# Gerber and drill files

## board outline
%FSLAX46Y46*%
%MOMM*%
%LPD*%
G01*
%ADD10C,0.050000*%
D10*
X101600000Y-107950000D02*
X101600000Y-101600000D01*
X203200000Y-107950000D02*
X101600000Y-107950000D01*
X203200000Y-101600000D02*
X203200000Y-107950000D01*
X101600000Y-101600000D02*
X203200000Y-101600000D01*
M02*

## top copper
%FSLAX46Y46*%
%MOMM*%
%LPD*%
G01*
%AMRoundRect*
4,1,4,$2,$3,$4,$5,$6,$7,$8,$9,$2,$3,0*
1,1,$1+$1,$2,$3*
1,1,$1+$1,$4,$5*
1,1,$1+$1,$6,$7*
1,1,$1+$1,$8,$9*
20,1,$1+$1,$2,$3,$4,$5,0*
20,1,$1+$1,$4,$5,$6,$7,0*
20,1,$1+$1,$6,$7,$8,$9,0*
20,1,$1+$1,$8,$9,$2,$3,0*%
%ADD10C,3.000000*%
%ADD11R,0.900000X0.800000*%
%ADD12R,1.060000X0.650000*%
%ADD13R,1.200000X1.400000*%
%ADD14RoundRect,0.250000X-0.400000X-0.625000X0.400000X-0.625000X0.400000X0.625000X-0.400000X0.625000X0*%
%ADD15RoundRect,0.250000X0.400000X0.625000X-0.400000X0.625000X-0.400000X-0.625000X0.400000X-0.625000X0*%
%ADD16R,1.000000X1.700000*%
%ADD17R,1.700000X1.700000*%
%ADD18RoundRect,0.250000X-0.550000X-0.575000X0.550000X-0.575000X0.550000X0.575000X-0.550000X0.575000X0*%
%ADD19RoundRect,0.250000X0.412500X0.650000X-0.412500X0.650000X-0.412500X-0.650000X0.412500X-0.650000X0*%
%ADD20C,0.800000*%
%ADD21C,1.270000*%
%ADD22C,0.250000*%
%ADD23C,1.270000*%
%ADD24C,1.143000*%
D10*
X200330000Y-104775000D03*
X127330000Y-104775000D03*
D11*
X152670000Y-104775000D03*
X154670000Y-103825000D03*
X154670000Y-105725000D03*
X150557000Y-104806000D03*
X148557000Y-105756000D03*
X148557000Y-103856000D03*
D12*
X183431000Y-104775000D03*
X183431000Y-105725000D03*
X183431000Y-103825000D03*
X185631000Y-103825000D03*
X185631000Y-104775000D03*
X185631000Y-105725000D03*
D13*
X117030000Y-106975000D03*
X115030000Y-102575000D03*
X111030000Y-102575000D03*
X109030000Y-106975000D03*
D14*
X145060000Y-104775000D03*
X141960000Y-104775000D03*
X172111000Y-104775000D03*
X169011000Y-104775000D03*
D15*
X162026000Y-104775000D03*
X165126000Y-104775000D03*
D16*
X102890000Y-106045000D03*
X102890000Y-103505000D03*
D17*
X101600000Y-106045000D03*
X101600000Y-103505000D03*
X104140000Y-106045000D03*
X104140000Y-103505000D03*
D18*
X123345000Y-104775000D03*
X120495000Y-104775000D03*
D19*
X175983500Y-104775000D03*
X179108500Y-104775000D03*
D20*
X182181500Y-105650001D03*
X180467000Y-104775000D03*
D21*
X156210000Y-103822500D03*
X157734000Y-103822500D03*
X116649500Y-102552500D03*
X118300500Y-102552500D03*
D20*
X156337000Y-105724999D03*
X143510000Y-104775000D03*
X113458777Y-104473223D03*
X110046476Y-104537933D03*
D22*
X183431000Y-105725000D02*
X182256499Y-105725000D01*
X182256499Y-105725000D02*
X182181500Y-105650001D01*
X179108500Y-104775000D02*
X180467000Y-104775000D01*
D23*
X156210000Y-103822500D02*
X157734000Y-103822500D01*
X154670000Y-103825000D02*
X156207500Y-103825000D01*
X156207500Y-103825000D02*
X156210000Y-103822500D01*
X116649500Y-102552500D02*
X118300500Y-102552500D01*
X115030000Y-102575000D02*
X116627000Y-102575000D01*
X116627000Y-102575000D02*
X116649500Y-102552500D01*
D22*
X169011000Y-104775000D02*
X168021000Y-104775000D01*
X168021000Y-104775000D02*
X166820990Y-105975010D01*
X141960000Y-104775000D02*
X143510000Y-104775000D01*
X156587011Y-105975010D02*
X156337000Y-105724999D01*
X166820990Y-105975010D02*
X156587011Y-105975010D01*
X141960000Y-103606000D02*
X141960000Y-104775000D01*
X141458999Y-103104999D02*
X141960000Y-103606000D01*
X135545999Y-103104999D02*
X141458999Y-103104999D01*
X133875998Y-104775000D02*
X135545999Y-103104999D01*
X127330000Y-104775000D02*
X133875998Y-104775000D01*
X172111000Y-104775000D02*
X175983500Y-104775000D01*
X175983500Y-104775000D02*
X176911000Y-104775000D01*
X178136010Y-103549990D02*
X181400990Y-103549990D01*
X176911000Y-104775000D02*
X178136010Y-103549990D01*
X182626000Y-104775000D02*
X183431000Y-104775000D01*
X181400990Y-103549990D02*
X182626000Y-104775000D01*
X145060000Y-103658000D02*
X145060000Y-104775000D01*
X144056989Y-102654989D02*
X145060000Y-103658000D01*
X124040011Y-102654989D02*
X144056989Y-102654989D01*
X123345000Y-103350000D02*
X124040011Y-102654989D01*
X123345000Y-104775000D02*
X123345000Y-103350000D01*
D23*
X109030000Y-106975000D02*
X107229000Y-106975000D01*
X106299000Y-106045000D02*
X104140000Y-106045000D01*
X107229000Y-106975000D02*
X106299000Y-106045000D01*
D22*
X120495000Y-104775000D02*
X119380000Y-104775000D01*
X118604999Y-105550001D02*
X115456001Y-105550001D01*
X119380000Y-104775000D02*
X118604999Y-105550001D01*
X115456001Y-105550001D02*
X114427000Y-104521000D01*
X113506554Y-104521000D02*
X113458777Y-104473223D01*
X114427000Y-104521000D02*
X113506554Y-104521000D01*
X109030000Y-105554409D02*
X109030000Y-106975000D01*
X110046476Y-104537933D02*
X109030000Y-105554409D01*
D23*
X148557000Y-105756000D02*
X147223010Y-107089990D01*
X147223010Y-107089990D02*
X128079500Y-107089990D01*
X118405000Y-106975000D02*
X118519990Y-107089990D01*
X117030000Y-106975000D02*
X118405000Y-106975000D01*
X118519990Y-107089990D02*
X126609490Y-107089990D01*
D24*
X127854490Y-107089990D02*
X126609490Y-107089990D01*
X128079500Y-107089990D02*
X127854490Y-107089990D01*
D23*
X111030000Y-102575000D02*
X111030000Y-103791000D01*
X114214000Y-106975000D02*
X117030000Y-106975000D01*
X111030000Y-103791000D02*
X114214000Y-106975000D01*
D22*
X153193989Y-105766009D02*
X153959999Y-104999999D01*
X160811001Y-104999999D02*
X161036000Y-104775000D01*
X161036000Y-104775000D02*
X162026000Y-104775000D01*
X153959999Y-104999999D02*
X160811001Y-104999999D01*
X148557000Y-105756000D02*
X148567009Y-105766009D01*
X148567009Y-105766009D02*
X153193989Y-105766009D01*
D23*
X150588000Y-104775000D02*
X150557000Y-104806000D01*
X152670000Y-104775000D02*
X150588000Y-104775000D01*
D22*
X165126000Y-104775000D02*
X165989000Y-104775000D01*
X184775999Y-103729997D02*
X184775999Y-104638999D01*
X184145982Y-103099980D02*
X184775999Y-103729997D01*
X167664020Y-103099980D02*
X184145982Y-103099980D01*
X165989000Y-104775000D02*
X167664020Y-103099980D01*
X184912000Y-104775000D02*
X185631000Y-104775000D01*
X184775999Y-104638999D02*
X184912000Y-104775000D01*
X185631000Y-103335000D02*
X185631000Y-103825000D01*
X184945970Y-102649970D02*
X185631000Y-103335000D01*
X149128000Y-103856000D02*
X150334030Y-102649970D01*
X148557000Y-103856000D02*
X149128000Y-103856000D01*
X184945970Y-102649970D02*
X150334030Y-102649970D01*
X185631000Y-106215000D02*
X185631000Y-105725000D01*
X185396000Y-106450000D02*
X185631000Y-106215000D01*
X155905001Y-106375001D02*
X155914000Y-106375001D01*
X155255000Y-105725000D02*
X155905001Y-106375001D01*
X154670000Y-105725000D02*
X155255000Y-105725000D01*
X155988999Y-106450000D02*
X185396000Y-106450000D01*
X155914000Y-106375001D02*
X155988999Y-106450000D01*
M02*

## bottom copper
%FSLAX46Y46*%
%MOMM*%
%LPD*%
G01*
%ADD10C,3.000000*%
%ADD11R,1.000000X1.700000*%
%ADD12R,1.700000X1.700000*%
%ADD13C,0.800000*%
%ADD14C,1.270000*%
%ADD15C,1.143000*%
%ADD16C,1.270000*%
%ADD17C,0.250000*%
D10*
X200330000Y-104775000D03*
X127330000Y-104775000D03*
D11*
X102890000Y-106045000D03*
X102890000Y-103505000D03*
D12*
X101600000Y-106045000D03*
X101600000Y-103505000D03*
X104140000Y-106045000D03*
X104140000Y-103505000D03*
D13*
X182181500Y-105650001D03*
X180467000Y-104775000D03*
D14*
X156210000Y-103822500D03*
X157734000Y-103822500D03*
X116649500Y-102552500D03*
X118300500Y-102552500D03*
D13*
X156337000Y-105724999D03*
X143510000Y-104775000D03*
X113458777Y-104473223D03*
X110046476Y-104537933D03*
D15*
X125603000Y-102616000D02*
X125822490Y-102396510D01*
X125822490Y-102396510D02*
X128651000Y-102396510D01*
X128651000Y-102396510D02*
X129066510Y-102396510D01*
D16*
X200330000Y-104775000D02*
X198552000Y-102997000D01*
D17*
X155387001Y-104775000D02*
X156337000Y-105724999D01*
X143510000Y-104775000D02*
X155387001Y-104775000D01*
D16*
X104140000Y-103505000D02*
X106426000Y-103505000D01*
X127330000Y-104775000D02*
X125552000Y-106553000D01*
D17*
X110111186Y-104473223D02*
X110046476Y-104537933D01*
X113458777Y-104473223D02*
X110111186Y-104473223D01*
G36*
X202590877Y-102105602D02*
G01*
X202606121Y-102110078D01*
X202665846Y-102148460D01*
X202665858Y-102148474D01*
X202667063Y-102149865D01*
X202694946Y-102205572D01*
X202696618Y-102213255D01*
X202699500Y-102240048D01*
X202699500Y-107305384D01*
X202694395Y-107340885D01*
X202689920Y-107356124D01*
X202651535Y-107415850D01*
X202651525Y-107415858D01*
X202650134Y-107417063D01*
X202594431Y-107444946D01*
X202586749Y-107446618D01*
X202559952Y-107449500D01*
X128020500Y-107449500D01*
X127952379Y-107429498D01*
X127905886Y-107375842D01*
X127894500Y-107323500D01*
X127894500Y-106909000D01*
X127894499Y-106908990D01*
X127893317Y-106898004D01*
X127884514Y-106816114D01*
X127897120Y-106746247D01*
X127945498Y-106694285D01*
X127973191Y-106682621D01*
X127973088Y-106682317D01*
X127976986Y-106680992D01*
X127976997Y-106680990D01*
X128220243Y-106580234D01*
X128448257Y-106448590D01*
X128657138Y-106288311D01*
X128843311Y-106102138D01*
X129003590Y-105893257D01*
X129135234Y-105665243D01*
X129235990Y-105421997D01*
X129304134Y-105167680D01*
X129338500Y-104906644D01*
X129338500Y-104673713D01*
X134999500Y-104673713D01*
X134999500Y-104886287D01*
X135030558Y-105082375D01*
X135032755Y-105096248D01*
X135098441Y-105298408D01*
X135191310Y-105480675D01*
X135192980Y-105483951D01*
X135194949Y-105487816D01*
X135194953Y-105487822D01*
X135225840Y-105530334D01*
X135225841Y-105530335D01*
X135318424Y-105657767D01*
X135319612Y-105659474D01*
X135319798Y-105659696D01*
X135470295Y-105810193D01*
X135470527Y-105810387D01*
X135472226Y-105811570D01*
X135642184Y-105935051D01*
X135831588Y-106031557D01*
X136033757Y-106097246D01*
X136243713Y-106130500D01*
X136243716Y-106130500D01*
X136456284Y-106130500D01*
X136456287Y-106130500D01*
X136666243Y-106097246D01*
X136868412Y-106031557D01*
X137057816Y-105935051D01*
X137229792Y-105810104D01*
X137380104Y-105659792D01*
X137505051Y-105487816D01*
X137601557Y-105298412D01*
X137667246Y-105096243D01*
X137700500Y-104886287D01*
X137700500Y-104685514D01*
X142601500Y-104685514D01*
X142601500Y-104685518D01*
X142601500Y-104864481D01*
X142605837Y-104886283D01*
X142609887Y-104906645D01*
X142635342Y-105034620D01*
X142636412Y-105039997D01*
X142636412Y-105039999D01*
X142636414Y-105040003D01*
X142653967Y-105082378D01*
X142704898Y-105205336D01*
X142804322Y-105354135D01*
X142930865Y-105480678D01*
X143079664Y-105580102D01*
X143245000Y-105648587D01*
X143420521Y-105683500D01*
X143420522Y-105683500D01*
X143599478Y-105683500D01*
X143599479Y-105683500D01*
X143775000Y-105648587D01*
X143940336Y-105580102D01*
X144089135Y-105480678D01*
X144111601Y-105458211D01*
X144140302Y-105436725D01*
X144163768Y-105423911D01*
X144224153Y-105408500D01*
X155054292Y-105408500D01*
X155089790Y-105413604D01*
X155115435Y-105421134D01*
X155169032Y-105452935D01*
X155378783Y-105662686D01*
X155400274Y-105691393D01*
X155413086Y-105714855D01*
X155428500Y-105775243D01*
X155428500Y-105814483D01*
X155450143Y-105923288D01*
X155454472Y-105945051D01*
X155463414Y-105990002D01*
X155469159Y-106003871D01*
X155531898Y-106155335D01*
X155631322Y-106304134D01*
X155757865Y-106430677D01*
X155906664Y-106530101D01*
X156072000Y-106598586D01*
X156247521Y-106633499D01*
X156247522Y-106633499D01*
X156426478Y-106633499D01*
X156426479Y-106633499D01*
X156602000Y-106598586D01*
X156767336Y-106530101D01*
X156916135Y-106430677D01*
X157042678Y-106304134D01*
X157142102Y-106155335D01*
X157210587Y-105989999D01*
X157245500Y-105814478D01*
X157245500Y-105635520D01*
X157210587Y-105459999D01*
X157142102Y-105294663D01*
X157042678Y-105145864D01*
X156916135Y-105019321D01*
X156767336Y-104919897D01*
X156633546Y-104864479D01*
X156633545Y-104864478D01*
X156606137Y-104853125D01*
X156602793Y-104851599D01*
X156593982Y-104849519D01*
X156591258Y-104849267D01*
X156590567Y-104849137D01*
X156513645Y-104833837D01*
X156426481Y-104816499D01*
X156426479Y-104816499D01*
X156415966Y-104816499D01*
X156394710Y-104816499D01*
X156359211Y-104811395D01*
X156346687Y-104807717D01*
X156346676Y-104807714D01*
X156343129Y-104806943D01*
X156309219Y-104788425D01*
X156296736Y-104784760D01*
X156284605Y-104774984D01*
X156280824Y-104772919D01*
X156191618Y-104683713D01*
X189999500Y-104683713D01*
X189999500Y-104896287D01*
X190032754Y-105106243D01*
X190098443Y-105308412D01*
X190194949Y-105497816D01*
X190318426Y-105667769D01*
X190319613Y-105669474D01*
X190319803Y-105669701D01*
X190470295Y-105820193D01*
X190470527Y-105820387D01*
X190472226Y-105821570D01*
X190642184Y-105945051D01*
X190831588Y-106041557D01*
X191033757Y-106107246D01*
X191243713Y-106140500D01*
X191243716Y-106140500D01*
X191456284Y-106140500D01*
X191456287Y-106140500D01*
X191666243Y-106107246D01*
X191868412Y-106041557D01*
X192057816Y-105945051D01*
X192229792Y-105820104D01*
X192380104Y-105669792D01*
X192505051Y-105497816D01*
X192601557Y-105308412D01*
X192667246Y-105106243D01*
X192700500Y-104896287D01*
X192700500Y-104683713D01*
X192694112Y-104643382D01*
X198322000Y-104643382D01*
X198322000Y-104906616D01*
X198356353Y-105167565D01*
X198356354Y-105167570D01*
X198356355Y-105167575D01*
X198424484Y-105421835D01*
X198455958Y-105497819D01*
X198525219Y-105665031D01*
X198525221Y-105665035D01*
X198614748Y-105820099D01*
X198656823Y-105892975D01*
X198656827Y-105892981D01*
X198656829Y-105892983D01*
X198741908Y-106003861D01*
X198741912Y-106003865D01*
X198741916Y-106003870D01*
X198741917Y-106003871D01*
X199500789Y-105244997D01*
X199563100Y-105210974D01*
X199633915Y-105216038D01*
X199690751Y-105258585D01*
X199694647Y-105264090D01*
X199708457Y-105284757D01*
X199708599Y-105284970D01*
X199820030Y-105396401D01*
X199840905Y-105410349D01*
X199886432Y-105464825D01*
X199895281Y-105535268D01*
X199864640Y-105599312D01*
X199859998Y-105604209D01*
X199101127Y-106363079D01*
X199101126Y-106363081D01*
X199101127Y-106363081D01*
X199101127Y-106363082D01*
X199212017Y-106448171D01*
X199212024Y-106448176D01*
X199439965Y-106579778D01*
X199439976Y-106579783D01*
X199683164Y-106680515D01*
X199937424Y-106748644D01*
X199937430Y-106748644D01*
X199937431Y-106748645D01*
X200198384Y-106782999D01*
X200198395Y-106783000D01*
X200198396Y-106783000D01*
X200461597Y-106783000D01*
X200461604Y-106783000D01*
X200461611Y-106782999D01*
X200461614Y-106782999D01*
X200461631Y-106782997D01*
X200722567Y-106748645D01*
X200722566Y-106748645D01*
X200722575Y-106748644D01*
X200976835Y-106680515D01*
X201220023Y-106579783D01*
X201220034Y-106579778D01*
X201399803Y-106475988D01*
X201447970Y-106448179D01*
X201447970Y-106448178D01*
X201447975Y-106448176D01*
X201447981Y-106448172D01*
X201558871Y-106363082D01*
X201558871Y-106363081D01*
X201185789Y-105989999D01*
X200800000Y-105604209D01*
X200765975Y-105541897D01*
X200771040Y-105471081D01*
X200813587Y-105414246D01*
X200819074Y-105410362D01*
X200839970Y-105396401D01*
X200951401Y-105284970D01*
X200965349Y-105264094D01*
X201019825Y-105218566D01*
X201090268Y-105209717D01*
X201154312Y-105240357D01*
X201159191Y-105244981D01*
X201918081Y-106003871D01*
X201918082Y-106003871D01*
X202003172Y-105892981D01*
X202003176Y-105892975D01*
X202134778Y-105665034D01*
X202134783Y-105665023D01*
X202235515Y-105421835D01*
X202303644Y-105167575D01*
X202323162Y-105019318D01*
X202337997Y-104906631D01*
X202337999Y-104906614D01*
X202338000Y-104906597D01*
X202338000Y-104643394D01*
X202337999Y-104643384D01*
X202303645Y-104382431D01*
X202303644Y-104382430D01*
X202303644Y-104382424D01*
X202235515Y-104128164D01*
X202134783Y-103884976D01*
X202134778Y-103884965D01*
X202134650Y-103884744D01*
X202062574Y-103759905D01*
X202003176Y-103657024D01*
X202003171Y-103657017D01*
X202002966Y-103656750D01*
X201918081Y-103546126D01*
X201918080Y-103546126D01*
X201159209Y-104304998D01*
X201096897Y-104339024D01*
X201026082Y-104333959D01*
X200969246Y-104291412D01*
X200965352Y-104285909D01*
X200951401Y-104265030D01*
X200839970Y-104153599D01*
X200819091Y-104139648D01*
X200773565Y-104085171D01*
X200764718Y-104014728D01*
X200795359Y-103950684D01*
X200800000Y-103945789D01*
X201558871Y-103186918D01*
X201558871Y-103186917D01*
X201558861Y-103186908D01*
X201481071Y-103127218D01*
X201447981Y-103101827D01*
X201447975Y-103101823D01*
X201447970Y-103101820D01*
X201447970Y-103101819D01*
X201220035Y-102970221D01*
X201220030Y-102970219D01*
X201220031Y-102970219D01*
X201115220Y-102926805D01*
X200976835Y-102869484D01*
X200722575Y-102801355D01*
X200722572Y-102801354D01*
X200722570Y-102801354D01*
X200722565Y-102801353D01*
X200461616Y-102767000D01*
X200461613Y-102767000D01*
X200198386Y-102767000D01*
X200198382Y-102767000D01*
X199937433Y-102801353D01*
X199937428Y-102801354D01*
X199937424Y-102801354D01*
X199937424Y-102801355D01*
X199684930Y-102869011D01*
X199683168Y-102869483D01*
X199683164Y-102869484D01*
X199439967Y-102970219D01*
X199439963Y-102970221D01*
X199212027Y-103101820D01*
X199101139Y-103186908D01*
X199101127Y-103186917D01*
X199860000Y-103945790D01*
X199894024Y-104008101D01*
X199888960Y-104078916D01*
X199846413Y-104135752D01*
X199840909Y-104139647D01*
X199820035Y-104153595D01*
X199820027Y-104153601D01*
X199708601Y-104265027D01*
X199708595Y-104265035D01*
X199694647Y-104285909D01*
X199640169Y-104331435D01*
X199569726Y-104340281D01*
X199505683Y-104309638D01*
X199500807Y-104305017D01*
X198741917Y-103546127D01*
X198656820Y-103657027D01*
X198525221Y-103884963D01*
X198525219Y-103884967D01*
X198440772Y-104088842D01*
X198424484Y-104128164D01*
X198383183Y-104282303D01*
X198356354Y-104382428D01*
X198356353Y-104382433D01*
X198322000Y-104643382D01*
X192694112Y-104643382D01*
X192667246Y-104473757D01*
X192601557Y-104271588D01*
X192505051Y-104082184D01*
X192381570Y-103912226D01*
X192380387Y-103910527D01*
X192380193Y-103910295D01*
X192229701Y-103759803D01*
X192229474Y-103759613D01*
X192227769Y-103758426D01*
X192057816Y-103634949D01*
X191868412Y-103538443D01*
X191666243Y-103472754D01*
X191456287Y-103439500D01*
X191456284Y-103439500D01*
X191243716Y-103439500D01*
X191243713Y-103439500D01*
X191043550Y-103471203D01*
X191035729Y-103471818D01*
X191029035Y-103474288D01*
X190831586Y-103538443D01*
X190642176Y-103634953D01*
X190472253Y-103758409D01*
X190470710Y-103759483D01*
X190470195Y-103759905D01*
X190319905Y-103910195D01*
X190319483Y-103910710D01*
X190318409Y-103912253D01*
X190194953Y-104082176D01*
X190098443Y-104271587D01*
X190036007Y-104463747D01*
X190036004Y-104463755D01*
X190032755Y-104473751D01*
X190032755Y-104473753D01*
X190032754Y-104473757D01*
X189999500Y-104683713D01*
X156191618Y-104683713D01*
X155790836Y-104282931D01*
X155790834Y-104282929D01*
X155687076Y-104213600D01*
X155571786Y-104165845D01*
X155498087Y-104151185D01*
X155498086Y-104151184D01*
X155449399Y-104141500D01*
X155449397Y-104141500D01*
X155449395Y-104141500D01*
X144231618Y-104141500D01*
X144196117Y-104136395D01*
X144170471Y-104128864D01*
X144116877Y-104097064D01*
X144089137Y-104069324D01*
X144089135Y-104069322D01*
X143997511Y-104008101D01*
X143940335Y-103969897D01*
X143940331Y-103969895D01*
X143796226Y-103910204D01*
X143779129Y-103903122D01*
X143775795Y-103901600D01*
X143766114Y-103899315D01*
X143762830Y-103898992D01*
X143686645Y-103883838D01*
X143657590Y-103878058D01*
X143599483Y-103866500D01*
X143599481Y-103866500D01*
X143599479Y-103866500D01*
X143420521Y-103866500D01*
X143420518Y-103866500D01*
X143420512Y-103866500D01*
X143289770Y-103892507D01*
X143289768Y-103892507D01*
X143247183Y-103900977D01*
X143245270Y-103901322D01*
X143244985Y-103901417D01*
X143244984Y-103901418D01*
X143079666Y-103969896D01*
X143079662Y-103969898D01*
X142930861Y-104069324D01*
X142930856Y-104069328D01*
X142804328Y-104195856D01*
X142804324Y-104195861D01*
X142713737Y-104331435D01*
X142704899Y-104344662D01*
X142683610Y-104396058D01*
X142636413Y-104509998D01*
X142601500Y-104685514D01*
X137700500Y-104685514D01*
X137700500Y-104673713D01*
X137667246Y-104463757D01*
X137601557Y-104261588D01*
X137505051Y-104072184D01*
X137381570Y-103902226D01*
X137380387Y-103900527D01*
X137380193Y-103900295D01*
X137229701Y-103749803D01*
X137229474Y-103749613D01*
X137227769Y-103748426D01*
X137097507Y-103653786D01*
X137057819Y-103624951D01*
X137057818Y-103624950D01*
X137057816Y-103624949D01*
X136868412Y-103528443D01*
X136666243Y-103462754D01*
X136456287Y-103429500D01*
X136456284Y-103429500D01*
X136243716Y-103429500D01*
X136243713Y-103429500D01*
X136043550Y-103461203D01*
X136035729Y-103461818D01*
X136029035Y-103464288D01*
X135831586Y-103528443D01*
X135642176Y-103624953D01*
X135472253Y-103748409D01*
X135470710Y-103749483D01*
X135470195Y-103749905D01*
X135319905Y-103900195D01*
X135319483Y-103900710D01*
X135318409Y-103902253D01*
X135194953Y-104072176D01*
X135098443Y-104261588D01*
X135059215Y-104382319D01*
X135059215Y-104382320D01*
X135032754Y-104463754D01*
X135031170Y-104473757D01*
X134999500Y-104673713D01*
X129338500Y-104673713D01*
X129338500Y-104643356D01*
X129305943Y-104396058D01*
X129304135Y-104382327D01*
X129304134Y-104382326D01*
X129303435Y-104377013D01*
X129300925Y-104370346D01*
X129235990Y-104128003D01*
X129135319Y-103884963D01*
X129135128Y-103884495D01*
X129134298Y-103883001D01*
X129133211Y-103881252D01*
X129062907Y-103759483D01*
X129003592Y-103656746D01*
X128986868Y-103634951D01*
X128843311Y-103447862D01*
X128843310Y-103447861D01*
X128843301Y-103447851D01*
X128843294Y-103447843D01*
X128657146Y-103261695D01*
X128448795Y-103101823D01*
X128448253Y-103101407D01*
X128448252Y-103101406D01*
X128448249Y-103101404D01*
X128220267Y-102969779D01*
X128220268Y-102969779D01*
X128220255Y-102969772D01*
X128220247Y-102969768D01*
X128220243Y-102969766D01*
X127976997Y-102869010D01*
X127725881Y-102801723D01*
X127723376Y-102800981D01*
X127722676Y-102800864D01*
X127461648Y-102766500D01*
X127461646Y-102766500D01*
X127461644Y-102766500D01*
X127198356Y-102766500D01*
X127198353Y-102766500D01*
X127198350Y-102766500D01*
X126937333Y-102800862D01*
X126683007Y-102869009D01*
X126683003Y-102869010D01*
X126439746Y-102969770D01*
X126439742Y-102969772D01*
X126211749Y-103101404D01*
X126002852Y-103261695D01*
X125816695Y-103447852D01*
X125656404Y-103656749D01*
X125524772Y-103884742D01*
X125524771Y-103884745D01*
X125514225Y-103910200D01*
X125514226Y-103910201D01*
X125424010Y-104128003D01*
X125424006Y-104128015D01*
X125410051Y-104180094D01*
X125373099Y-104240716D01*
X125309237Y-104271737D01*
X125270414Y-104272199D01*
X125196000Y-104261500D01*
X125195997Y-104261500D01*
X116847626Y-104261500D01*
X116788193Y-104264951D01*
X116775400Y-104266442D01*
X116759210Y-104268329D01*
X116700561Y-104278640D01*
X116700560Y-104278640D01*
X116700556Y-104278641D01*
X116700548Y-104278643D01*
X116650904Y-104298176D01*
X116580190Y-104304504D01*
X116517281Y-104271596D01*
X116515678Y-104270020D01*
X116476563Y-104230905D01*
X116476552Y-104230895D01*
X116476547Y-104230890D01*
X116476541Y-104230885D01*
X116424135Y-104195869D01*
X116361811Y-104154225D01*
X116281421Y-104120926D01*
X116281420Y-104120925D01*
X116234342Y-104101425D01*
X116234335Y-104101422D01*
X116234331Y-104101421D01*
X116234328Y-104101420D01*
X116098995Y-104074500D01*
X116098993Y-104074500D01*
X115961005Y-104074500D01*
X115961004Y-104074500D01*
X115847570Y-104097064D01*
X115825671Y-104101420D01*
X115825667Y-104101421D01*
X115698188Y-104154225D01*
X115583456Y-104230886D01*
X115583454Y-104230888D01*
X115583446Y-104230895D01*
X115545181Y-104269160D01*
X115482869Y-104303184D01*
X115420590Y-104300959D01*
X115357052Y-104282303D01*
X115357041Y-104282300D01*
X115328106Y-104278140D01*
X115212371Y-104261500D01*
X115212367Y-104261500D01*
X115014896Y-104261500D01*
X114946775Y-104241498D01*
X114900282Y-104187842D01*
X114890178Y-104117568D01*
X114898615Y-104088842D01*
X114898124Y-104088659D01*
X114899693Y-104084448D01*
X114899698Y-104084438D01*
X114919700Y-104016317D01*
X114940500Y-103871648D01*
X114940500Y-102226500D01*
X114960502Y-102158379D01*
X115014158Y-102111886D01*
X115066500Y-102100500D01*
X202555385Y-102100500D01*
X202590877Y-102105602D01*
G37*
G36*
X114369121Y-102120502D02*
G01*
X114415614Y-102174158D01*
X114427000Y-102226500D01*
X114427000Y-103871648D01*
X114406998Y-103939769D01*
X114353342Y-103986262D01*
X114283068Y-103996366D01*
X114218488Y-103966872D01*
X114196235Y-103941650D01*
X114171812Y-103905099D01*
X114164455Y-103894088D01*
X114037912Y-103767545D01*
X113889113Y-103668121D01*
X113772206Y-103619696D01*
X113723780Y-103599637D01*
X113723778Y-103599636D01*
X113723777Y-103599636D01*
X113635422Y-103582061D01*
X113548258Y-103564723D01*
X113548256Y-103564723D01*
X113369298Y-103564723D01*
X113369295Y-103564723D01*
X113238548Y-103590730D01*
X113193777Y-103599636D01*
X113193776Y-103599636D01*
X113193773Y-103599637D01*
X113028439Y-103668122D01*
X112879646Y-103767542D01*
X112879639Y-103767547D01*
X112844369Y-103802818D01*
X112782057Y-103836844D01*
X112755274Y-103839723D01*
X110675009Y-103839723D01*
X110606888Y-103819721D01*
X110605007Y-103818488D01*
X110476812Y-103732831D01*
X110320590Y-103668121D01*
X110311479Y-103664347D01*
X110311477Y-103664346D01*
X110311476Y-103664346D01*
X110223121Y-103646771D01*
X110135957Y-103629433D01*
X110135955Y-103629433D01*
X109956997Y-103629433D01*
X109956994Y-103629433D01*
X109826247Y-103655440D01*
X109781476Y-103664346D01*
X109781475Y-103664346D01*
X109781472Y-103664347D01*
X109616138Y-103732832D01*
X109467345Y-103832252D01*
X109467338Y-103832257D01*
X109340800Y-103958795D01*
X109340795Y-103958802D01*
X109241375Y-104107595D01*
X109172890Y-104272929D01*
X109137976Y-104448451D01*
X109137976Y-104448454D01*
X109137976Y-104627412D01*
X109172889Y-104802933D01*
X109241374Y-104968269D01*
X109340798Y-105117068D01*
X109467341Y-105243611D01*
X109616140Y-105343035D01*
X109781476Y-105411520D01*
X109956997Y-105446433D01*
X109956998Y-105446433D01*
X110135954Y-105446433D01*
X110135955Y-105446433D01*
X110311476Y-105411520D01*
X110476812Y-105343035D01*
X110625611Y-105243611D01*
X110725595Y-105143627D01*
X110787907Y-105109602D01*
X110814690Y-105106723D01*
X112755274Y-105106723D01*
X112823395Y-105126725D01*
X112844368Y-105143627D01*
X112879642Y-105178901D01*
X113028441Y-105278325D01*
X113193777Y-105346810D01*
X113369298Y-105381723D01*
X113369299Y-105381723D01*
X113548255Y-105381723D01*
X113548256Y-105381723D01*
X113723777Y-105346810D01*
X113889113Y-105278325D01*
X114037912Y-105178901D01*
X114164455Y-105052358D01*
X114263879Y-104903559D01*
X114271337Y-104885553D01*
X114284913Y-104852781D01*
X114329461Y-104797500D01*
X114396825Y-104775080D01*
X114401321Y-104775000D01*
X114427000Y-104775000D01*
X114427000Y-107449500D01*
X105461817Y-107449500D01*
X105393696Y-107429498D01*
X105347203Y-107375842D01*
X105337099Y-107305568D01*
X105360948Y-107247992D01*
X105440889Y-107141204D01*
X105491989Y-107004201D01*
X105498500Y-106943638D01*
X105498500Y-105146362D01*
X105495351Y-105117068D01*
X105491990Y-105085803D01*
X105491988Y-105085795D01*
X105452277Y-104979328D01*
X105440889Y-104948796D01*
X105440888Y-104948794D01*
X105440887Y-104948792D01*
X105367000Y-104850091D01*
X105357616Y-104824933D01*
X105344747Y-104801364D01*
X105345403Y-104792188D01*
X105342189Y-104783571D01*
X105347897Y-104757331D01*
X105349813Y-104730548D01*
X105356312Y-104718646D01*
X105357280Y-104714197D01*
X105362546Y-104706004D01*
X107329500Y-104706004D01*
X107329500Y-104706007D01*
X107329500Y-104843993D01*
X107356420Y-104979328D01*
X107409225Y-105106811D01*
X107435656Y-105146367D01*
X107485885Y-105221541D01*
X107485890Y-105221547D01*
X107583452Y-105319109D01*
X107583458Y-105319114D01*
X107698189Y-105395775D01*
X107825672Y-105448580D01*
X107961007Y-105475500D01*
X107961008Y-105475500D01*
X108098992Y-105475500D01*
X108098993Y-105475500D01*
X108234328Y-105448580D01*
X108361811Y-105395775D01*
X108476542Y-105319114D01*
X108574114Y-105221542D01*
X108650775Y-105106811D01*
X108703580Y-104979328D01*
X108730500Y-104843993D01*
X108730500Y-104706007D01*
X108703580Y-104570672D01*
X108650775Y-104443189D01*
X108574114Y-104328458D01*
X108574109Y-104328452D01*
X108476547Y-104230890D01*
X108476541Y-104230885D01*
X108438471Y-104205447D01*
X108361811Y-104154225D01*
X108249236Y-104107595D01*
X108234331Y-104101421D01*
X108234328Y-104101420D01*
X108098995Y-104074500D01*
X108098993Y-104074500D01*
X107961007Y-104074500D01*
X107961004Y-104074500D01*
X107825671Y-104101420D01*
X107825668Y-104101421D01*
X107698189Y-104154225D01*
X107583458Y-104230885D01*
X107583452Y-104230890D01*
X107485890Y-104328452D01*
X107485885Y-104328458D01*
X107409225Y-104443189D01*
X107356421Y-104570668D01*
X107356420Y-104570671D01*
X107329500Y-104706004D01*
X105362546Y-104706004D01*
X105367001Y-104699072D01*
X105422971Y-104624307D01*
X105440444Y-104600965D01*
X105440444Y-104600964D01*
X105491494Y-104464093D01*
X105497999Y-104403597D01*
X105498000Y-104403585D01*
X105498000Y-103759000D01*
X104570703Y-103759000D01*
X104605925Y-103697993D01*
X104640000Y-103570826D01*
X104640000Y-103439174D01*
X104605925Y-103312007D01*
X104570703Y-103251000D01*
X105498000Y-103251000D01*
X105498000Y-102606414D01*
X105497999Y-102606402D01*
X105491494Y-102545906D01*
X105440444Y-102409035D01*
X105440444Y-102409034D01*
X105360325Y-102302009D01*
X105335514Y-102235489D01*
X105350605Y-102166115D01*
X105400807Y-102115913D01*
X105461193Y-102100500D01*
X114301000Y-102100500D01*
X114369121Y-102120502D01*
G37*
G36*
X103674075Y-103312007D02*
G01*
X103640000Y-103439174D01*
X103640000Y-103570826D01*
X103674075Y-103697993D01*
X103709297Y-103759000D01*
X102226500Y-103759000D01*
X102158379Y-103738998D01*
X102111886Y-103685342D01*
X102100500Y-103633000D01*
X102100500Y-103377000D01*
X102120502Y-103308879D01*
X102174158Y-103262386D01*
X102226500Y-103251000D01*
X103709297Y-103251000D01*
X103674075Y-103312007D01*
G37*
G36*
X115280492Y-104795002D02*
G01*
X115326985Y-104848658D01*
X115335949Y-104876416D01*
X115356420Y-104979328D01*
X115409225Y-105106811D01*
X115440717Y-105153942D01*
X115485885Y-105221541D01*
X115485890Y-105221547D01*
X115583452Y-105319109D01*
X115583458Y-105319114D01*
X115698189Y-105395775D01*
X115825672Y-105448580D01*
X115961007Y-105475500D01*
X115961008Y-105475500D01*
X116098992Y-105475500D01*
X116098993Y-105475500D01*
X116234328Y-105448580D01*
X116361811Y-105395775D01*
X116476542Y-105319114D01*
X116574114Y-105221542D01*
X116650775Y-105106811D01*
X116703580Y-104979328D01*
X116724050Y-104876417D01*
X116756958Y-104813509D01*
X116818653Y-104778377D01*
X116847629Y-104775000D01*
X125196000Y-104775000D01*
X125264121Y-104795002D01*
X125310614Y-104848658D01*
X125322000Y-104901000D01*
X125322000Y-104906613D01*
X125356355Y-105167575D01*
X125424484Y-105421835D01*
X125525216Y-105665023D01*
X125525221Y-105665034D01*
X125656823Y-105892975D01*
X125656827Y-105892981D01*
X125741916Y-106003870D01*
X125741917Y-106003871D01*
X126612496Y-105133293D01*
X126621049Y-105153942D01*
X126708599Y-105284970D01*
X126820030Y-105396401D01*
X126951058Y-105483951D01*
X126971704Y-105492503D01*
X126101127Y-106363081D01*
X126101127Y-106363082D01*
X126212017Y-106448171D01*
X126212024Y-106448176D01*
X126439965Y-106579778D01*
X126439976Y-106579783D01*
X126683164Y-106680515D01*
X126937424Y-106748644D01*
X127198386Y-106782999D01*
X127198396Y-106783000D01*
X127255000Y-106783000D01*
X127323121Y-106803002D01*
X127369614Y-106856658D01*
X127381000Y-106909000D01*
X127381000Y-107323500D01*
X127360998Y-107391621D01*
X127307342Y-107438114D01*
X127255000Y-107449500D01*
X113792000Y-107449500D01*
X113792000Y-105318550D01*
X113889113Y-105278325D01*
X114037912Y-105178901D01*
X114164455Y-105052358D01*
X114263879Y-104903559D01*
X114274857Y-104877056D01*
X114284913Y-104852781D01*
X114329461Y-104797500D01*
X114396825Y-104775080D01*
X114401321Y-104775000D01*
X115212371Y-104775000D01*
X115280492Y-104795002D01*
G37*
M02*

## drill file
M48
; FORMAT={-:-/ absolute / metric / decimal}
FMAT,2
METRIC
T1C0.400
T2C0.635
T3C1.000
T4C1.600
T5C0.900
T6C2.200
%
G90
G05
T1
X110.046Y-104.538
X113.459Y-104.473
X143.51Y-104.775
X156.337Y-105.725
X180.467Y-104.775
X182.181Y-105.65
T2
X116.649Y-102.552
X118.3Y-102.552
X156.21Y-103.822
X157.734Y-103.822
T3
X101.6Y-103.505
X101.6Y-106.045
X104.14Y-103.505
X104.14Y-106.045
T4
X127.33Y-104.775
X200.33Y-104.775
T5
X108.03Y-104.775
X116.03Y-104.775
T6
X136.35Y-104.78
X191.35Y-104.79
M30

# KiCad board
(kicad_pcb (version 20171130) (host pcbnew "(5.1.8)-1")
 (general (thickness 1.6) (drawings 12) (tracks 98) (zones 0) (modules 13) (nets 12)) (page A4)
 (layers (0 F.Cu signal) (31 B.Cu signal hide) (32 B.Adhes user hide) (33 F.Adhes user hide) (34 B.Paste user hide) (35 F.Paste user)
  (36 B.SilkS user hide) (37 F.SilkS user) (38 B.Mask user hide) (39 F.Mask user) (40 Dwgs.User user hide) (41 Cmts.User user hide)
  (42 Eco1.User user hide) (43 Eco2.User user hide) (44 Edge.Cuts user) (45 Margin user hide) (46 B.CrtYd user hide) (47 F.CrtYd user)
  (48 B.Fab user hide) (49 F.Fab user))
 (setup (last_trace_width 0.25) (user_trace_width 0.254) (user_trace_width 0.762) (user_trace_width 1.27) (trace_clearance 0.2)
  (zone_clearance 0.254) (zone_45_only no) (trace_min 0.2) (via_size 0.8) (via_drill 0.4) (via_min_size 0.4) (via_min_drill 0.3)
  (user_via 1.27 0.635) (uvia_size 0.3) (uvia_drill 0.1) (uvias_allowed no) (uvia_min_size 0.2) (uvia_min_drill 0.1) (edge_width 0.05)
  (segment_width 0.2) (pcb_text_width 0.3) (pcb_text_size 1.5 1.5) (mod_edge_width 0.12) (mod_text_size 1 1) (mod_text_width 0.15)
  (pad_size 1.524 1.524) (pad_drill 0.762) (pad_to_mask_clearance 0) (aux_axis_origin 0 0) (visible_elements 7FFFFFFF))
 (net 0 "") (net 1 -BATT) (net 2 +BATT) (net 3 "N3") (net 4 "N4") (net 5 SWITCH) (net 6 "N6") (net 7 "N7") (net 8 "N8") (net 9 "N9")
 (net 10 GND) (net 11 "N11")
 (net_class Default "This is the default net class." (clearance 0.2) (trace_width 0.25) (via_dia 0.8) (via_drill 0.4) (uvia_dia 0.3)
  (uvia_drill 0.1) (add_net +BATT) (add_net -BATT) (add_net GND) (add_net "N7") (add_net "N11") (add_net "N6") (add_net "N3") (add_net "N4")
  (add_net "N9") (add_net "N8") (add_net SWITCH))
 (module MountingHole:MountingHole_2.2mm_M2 (layer F.Cu) (at 191.35 104.79)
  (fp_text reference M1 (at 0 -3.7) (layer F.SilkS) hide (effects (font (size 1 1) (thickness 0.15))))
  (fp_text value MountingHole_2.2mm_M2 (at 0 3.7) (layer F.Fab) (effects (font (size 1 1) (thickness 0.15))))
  (pad 1 np_thru_hole circle (at 0 0) (size 2.2 2.2) (drill 2.2) (layers *.Cu *.Mask)))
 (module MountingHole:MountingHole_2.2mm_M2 (layer F.Cu) (at 136.35 104.78)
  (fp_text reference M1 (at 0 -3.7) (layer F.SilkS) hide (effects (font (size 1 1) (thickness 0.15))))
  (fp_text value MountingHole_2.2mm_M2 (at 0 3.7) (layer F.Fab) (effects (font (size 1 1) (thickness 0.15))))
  (pad 1 np_thru_hole circle (at 0 0) (size 2.2 2.2) (drill 2.2) (layers *.Cu *.Mask)))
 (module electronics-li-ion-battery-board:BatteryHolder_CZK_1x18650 (layer F.Cu) (at 163.83 104.775)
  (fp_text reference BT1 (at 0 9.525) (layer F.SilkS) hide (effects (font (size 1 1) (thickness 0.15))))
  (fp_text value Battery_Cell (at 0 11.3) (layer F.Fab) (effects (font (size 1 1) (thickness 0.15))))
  (pad 2 thru_hole circle (at 36.5 0) (size 3 3) (drill 1.6) (layers *.Cu *.Mask) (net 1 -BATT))
  (pad 1 thru_hole circle (at -36.5 0) (size 3 3) (drill 1.6) (layers *.Cu *.Mask) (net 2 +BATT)))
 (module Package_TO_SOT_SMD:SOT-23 (layer F.Cu) (at 153.67 104.775 180)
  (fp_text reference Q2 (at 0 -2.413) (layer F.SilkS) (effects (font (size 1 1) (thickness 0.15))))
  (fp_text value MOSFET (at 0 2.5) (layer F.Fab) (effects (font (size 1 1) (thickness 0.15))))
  (pad 3 smd rect (at 1 0 180) (size 0.9 0.8) (layers F.Cu F.Paste F.Mask) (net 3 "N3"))
  (pad 2 smd rect (at -1 0.95 180) (size 0.9 0.8) (layers F.Cu F.Paste F.Mask) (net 1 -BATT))
  (pad 1 smd rect (at -1 -0.95 180) (size 0.9 0.8) (layers F.Cu F.Paste F.Mask) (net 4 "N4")))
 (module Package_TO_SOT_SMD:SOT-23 (layer F.Cu) (at 149.557 104.806)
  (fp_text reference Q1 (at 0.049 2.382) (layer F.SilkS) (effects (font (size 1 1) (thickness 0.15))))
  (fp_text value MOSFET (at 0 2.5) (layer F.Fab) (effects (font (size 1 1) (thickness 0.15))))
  (pad 3 smd rect (at 1 0) (size 0.9 0.8) (layers F.Cu F.Paste F.Mask) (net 3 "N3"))
  (pad 2 smd rect (at -1 0.95) (size 0.9 0.8) (layers F.Cu F.Paste F.Mask) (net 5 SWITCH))
  (pad 1 smd rect (at -1 -0.95) (size 0.9 0.8) (layers F.Cu F.Paste F.Mask) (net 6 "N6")))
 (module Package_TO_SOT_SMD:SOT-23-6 (layer F.Cu) (at 184.531 104.775 180)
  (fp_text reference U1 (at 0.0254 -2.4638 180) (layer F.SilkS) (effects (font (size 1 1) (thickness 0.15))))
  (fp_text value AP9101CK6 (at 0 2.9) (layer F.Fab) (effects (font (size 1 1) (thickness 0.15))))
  (pad 5 smd rect (at 1.1 0 180) (size 1.06 0.65) (layers F.Cu F.Paste F.Mask) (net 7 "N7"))
  (pad 6 smd rect (at 1.1 -0.95 180) (size 1.06 0.65) (layers F.Cu F.Paste F.Mask) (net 1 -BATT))
  (pad 4 smd rect (at 1.1 0.95 180) (size 1.06 0.65) (layers F.Cu F.Paste F.Mask) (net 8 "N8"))
  (pad 3 smd rect (at -1.1 0.95 180) (size 1.06 0.65) (layers F.Cu F.Paste F.Mask) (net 6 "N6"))
  (pad 2 smd rect (at -1.1 0 180) (size 1.06 0.65) (layers F.Cu F.Paste F.Mask) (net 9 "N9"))
  (pad 1 smd rect (at -1.1 -0.95 180) (size 1.06 0.65) (layers F.Cu F.Paste F.Mask) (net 4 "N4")))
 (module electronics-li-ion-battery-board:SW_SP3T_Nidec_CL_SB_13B (layer F.Cu) (at 113.03 104.775 180)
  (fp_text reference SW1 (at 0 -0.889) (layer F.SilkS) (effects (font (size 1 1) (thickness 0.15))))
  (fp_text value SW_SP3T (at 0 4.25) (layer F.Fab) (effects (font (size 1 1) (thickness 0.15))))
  (pad "" np_thru_hole circle (at -3 0 180) (size 0.9 0.9) (drill 0.9) (layers *.Cu *.Mask))
  (pad "" np_thru_hole circle (at 5 0 180) (size 0.9 0.9) (drill 0.9) (layers *.Cu *.Mask))
  (pad 1 smd rect (at -4 -2.2 180) (size 1.2 1.4) (layers F.Cu F.Paste F.Mask) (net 5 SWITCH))
  (pad 2 smd rect (at -2 2.2 180) (size 1.2 1.4) (layers F.Cu F.Paste F.Mask) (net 1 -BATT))
  (pad 3 smd rect (at 2 2.2 180) (size 1.2 1.4) (layers F.Cu F.Paste F.Mask) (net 5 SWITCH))
  (pad 4 smd rect (at 4 -2.2 180) (size 1.2 1.4) (layers F.Cu F.Paste F.Mask) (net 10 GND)))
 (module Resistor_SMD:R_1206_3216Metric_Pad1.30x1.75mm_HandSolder (layer F.Cu) (at 143.51 104.775)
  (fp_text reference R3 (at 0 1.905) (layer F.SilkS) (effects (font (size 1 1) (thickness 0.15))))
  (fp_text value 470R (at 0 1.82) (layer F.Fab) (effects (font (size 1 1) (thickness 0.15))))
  (pad 2 smd roundrect (at 1.55 0) (size 1.3 1.75) (layers F.Cu F.Paste F.Mask) (roundrect_rratio 0.192308) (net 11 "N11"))
  (pad 1 smd roundrect (at -1.55 0) (size 1.3 1.75) (layers F.Cu F.Paste F.Mask) (roundrect_rratio 0.192308) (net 2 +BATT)))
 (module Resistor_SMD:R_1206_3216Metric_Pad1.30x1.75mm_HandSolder (layer F.Cu) (at 170.561 104.775)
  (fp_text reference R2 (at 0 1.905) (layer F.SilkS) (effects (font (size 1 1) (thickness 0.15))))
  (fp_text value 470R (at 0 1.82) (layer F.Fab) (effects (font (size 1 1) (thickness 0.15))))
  (pad 2 smd roundrect (at 1.55 0) (size 1.3 1.75) (layers F.Cu F.Paste F.Mask) (roundrect_rratio 0.192308) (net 7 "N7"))
  (pad 1 smd roundrect (at -1.55 0) (size 1.3 1.75) (layers F.Cu F.Paste F.Mask) (roundrect_rratio 0.192308) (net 2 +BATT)))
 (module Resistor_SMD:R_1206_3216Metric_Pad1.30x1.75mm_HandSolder (layer F.Cu) (at 163.576 104.775 180)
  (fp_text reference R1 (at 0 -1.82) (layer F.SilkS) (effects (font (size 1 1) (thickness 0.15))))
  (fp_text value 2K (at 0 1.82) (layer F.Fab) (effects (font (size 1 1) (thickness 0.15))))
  (pad 2 smd roundrect (at 1.55 0 180) (size 1.3 1.75) (layers F.Cu F.Paste F.Mask) (roundrect_rratio 0.192308) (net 5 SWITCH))
  (pad 1 smd roundrect (at -1.55 0 180) (size 1.3 1.75) (layers F.Cu F.Paste F.Mask) (roundrect_rratio 0.192308) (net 9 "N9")))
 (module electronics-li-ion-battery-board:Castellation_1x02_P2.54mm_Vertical (layer B.Cu) (at 104.14 103.505 180)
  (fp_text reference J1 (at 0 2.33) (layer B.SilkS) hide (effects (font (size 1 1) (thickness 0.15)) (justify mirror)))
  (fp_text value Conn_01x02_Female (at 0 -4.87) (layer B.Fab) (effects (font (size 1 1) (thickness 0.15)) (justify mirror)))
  (pad 2 smd rect (at 1.25 -2.54 180) (size 1 1.7) (layers F.Cu F.Paste F.Mask) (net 10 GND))
  (pad 1 smd rect (at 1.25 0 180) (size 1 1.7) (layers F.Cu F.Paste F.Mask) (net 2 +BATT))
  (pad 2 smd rect (at 1.25 -2.54 180) (size 1 1.7) (layers B.Cu B.Paste) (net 10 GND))
  (pad 1 smd rect (at 1.25 0 180) (size 1 1.7) (layers B.Cu B.Paste B.Mask) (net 2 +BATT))
  (pad 2 thru_hole rect (at 2.54 -2.54 180) (size 1.7 1.7) (drill 1) (layers *.Cu *.Mask) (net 10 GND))
  (pad 1 thru_hole rect (at 2.54 0 180) (size 1.7 1.7) (drill 1) (layers *.Cu *.Mask) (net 2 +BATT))
  (pad 2 thru_hole rect (at 0 -2.54 180) (size 1.7 1.7) (drill 1) (layers *.Cu *.Mask) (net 10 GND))
  (pad 1 thru_hole rect (at 0 0 180) (size 1.7 1.7) (drill 1) (layers *.Cu *.Mask) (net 2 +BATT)))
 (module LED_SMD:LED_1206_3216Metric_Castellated (layer F.Cu) (at 121.92 104.775)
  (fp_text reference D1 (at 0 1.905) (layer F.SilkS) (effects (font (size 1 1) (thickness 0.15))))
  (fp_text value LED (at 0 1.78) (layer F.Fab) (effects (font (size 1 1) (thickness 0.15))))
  (pad 2 smd roundrect (at 1.425 0) (size 1.6 1.65) (layers F.Cu F.Paste F.Mask) (roundrect_rratio 0.15625) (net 11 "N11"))
  (pad 1 smd roundrect (at -1.425 0) (size 1.6 1.65) (layers F.Cu F.Paste F.Mask) (roundrect_rratio 0.15625) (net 10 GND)))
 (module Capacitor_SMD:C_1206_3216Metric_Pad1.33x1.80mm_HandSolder (layer F.Cu) (at 177.546 104.775 180)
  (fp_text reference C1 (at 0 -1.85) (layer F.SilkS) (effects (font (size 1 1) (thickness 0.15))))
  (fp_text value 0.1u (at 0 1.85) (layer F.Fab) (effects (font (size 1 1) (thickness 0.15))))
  (pad 2 smd roundrect (at 1.5625 0 180) (size 1.325 1.8) (layers F.Cu F.Paste F.Mask) (roundrect_rratio 0.188679) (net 7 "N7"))
  (pad 1 smd roundrect (at -1.5625 0 180) (size 1.325 1.8) (layers F.Cu F.Paste F.Mask) (roundrect_rratio 0.188679) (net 1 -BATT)))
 (gr_line (start 101.6 107.95) (end 101.6 101.6) (layer Edge.Cuts) (width 0.05))
 (gr_line (start 203.2 107.95) (end 101.6 107.95) (layer Edge.Cuts) (width 0.05))
 (gr_line (start 203.2 101.6) (end 203.2 107.95) (layer Edge.Cuts) (width 0.05))
 (gr_line (start 101.6 101.6) (end 203.2 101.6) (layer Edge.Cuts) (width 0.05))
 (segment (start 125.603 102.616) (end 125.82249 102.39651) (width 1.143) (layer B.Cu) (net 1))
 (segment (start 125.82249 102.39651) (end 128.651 102.39651) (width 1.143) (layer B.Cu) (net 1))
 (segment (start 128.651 102.39651) (end 129.06651 102.39651) (width 1.143) (layer B.Cu) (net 1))
 (via (at 182.1815 105.650001) (size 0.8) (drill 0.4) (layers F.Cu B.Cu) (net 1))
 (segment (start 183.431 105.725) (end 182.256499 105.725) (width 0.25) (layer F.Cu) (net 1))
 (segment (start 182.256499 105.725) (end 182.1815 105.650001) (width 0.25) (layer F.Cu) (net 1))
 (via (at 180.467 104.775) (size 0.8) (drill 0.4) (layers F.Cu B.Cu) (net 1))
 (segment (start 179.1085 104.775) (end 180.467 104.775) (width 0.25) (layer F.Cu) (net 1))
 (via (at 156.21 103.8225) (size 1.27) (drill 0.635) (layers F.Cu B.Cu) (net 1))
 (segment (start 156.21 103.8225) (end 157.734 103.8225) (width 1.27) (layer F.Cu) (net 1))
 (via (at 157.734 103.8225) (size 1.27) (drill 0.635) (layers F.Cu B.Cu) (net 1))
 (segment (start 154.67 103.825) (end 156.2075 103.825) (width 1.27) (layer F.Cu) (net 1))
 (segment (start 156.2075 103.825) (end 156.21 103.8225) (width 1.27) (layer F.Cu) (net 1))
 (via (at 116.6495 102.5525) (size 1.27) (drill 0.635) (layers F.Cu B.Cu) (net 1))
 (segment (start 116.6495 102.5525) (end 118.3005 102.5525) (width 1.27) (layer F.Cu) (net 1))
 (via (at 118.3005 102.5525) (size 1.27) (drill 0.635) (layers F.Cu B.Cu) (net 1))
 (segment (start 115.03 102.575) (end 116.627 102.575) (width 1.27) (layer F.Cu) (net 1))
 (segment (start 116.627 102.575) (end 116.6495 102.5525) (width 1.27) (layer F.Cu) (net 1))
 (segment (start 200.33 104.775) (end 198.552 102.997) (width 1.27) (layer B.Cu) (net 1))
 (segment (start 169.011 104.775) (end 168.021 104.775) (width 0.25) (layer F.Cu) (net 2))
 (via (at 156.337 105.724999) (size 0.8) (drill 0.4) (layers F.Cu B.Cu) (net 2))
 (segment (start 168.021 104.775) (end 166.82099 105.97501) (width 0.25) (layer F.Cu) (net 2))
 (segment (start 155.387001 104.775) (end 156.337 105.724999) (width 0.25) (layer B.Cu) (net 2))
 (via (at 143.51 104.775) (size 0.8) (drill 0.4) (layers F.Cu B.Cu) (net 2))
 (segment (start 141.96 104.775) (end 143.51 104.775) (width 0.25) (layer F.Cu) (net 2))
 (segment (start 143.51 104.775) (end 155.387001 104.775) (width 0.25) (layer B.Cu) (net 2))
 (segment (start 156.587011 105.97501) (end 156.337 105.724999) (width 0.25) (layer F.Cu) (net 2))
 (segment (start 166.82099 105.97501) (end 156.587011 105.97501) (width 0.25) (layer F.Cu) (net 2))
 (segment (start 104.14 103.505) (end 106.426 103.505) (width 1.27) (layer B.Cu) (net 2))
 (segment (start 127.33 104.775) (end 125.552 106.553) (width 1.27) (layer B.Cu) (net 2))
 (segment (start 141.96 103.606) (end 141.96 104.775) (width 0.25) (layer F.Cu) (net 2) (status 1000000))
 (segment (start 141.458999 103.104999) (end 141.96 103.606) (width 0.25) (layer F.Cu) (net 2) (status 1000000))
 (segment (start 135.545999 103.104999) (end 141.458999 103.104999) (width 0.25) (layer F.Cu) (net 2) (status 1000000))
 (segment (start 133.875998 104.775) (end 135.545999 103.104999) (width 0.25) (layer F.Cu) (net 2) (status 1000000))
 (segment (start 127.33 104.775) (end 133.875998 104.775) (width 0.25) (layer F.Cu) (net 2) (status 1000000))
 (segment (start 172.111 104.775) (end 175.9835 104.775) (width 0.25) (layer F.Cu) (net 7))
 (segment (start 175.9835 104.775) (end 176.911 104.775) (width 0.25) (layer F.Cu) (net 7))
 (segment (start 178.13601 103.54999) (end 181.40099 103.54999) (width 0.25) (layer F.Cu) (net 7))
 (segment (start 176.911 104.775) (end 178.13601 103.54999) (width 0.25) (layer F.Cu) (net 7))
 (segment (start 182.626 104.775) (end 183.431 104.775) (width 0.25) (layer F.Cu) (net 7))
 (segment (start 181.40099 103.54999) (end 182.626 104.775) (width 0.25) (layer F.Cu) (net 7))
 (segment (start 145.06 103.658) (end 145.06 104.775) (width 0.25) (layer F.Cu) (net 11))
 (segment (start 144.056989 102.654989) (end 145.06 103.658) (width 0.25) (layer F.Cu) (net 11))
 (segment (start 124.040011 102.654989) (end 144.056989 102.654989) (width 0.25) (layer F.Cu) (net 11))
 (segment (start 123.345 103.35) (end 124.040011 102.654989) (width 0.25) (layer F.Cu) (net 11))
 (segment (start 123.345 104.775) (end 123.345 103.35) (width 0.25) (layer F.Cu) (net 11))
 (segment (start 109.03 106.975) (end 107.229 106.975) (width 1.27) (layer F.Cu) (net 10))
 (segment (start 106.299 106.045) (end 104.14 106.045) (width 1.27) (layer F.Cu) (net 10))
 (segment (start 107.229 106.975) (end 106.299 106.045) (width 1.27) (layer F.Cu) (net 10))
 (segment (start 120.495 104.775) (end 119.38 104.775) (width 0.25) (layer F.Cu) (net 10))
 (segment (start 118.604999 105.550001) (end 115.456001 105.550001) (width 0.25) (layer F.Cu) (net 10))
 (segment (start 119.38 104.775) (end 118.604999 105.550001) (width 0.25) (layer F.Cu) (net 10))
 (segment (start 115.456001 105.550001) (end 114.427 104.521) (width 0.25) (layer F.Cu) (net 10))
 (via (at 113.458777 104.473223) (size 0.8) (drill 0.4) (layers F.Cu B.Cu) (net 10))
 (segment (start 113.506554 104.521) (end 113.458777 104.473223) (width 0.25) (layer F.Cu) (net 10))
 (segment (start 114.427 104.521) (end 113.506554 104.521) (width 0.25) (layer F.Cu) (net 10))
 (via (at 110.046476 104.537933) (size 0.8) (drill 0.4) (layers F.Cu B.Cu) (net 10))
 (segment (start 110.111186 104.473223) (end 110.046476 104.537933) (width 0.25) (layer B.Cu) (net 10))
 (segment (start 113.458777 104.473223) (end 110.111186 104.473223) (width 0.25) (layer B.Cu) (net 10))
 (segment (start 109.03 105.554409) (end 109.03 106.975) (width 0.25) (layer F.Cu) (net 10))
 (segment (start 110.046476 104.537933) (end 109.03 105.554409) (width 0.25) (layer F.Cu) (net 10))
 (segment (start 148.557 105.756) (end 147.22301 107.08999) (width 1.27) (layer F.Cu) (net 5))
 (segment (start 147.22301 107.08999) (end 128.0795 107.08999) (width 1.27) (layer F.Cu) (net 5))
 (segment (start 118.405 106.975) (end 118.51999 107.08999) (width 1.27) (layer F.Cu) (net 5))
 (segment (start 117.03 106.975) (end 118.405 106.975) (width 1.27) (layer F.Cu) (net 5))
 (segment (start 118.51999 107.08999) (end 126.60949 107.08999) (width 1.27) (layer F.Cu) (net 5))
 (segment (start 127.85449 107.08999) (end 126.60949 107.08999) (width 1.143) (layer F.Cu) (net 5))
 (segment (start 128.0795 107.08999) (end 127.85449 107.08999) (width 1.143) (layer F.Cu) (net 5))
 (segment (start 111.03 102.575) (end 111.03 103.791) (width 1.27) (layer F.Cu) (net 5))
 (segment (start 114.214 106.975) (end 117.03 106.975) (width 1.27) (layer F.Cu) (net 5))
 (segment (start 111.03 103.791) (end 114.214 106.975) (width 1.27) (layer F.Cu) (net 5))
 (segment (start 153.193989 105.766009) (end 153.959999 104.999999) (width 0.25) (layer F.Cu) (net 5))
 (segment (start 160.811001 104.999999) (end 161.036 104.775) (width 0.25) (layer F.Cu) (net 5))
 (segment (start 161.036 104.775) (end 162.026 104.775) (width 0.25) (layer F.Cu) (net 5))
 (segment (start 153.959999 104.999999) (end 160.811001 104.999999) (width 0.25) (layer F.Cu) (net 5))
 (segment (start 148.557 105.756) (end 148.567009 105.766009) (width 0.25) (layer F.Cu) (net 5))
 (segment (start 148.567009 105.766009) (end 153.193989 105.766009) (width 0.25) (layer F.Cu) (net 5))
 (segment (start 150.588 104.775) (end 150.557 104.806) (width 1.27) (layer F.Cu) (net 3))
 (segment (start 152.67 104.775) (end 150.588 104.775) (width 1.27) (layer F.Cu) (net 3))
 (segment (start 165.126 104.775) (end 165.989 104.775) (width 0.25) (layer F.Cu) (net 9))
 (segment (start 184.775999 103.729997) (end 184.775999 104.638999) (width 0.25) (layer F.Cu) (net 9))
 (segment (start 184.145982 103.09998) (end 184.775999 103.729997) (width 0.25) (layer F.Cu) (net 9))
 (segment (start 167.66402 103.09998) (end 184.145982 103.09998) (width 0.25) (layer F.Cu) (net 9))
 (segment (start 165.989 104.775) (end 167.66402 103.09998) (width 0.25) (layer F.Cu) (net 9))
 (segment (start 184.912 104.775) (end 185.631 104.775) (width 0.25) (layer F.Cu) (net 9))
 (segment (start 184.775999 104.638999) (end 184.912 104.775) (width 0.25) (layer F.Cu) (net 9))
 (segment (start 185.631 103.335) (end 185.631 103.825) (width 0.25) (layer F.Cu) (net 6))
 (segment (start 184.94597 102.64997) (end 185.631 103.335) (width 0.25) (layer F.Cu) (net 6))
 (segment (start 149.128 103.856) (end 150.33403 102.64997) (width 0.25) (layer F.Cu) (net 6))
 (segment (start 148.557 103.856) (end 149.128 103.856) (width 0.25) (layer F.Cu) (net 6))
 (segment (start 184.94597 102.64997) (end 150.33403 102.64997) (width 0.25) (layer F.Cu) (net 6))
 (segment (start 185.631 106.215) (end 185.631 105.725) (width 0.25) (layer F.Cu) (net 4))
 (segment (start 185.396 106.45) (end 185.631 106.215) (width 0.25) (layer F.Cu) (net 4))
 (segment (start 155.905001 106.375001) (end 155.914 106.375001) (width 0.25) (layer F.Cu) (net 4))
 (segment (start 155.255 105.725) (end 155.905001 106.375001) (width 0.25) (layer F.Cu) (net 4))
 (segment (start 154.67 105.725) (end 155.255 105.725) (width 0.25) (layer F.Cu) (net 4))
 (segment (start 155.988999 106.45) (end 185.396 106.45) (width 0.25) (layer F.Cu) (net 4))
 (segment (start 155.914 106.375001) (end 155.988999 106.45) (width 0.25) (layer F.Cu) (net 4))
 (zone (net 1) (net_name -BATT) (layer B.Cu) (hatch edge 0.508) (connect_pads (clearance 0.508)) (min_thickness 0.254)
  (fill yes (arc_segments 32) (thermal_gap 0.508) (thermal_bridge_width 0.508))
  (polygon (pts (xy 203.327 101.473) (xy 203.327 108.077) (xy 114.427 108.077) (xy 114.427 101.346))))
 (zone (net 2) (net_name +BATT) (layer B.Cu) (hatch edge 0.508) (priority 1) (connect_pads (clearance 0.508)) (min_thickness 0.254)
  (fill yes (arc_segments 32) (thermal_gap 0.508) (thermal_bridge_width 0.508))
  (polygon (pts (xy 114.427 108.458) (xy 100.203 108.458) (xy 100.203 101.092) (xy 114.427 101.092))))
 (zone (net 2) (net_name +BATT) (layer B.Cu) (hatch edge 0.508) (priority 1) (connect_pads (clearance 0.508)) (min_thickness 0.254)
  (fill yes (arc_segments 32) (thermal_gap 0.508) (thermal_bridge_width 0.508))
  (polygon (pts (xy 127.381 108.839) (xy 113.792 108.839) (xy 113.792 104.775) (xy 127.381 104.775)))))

